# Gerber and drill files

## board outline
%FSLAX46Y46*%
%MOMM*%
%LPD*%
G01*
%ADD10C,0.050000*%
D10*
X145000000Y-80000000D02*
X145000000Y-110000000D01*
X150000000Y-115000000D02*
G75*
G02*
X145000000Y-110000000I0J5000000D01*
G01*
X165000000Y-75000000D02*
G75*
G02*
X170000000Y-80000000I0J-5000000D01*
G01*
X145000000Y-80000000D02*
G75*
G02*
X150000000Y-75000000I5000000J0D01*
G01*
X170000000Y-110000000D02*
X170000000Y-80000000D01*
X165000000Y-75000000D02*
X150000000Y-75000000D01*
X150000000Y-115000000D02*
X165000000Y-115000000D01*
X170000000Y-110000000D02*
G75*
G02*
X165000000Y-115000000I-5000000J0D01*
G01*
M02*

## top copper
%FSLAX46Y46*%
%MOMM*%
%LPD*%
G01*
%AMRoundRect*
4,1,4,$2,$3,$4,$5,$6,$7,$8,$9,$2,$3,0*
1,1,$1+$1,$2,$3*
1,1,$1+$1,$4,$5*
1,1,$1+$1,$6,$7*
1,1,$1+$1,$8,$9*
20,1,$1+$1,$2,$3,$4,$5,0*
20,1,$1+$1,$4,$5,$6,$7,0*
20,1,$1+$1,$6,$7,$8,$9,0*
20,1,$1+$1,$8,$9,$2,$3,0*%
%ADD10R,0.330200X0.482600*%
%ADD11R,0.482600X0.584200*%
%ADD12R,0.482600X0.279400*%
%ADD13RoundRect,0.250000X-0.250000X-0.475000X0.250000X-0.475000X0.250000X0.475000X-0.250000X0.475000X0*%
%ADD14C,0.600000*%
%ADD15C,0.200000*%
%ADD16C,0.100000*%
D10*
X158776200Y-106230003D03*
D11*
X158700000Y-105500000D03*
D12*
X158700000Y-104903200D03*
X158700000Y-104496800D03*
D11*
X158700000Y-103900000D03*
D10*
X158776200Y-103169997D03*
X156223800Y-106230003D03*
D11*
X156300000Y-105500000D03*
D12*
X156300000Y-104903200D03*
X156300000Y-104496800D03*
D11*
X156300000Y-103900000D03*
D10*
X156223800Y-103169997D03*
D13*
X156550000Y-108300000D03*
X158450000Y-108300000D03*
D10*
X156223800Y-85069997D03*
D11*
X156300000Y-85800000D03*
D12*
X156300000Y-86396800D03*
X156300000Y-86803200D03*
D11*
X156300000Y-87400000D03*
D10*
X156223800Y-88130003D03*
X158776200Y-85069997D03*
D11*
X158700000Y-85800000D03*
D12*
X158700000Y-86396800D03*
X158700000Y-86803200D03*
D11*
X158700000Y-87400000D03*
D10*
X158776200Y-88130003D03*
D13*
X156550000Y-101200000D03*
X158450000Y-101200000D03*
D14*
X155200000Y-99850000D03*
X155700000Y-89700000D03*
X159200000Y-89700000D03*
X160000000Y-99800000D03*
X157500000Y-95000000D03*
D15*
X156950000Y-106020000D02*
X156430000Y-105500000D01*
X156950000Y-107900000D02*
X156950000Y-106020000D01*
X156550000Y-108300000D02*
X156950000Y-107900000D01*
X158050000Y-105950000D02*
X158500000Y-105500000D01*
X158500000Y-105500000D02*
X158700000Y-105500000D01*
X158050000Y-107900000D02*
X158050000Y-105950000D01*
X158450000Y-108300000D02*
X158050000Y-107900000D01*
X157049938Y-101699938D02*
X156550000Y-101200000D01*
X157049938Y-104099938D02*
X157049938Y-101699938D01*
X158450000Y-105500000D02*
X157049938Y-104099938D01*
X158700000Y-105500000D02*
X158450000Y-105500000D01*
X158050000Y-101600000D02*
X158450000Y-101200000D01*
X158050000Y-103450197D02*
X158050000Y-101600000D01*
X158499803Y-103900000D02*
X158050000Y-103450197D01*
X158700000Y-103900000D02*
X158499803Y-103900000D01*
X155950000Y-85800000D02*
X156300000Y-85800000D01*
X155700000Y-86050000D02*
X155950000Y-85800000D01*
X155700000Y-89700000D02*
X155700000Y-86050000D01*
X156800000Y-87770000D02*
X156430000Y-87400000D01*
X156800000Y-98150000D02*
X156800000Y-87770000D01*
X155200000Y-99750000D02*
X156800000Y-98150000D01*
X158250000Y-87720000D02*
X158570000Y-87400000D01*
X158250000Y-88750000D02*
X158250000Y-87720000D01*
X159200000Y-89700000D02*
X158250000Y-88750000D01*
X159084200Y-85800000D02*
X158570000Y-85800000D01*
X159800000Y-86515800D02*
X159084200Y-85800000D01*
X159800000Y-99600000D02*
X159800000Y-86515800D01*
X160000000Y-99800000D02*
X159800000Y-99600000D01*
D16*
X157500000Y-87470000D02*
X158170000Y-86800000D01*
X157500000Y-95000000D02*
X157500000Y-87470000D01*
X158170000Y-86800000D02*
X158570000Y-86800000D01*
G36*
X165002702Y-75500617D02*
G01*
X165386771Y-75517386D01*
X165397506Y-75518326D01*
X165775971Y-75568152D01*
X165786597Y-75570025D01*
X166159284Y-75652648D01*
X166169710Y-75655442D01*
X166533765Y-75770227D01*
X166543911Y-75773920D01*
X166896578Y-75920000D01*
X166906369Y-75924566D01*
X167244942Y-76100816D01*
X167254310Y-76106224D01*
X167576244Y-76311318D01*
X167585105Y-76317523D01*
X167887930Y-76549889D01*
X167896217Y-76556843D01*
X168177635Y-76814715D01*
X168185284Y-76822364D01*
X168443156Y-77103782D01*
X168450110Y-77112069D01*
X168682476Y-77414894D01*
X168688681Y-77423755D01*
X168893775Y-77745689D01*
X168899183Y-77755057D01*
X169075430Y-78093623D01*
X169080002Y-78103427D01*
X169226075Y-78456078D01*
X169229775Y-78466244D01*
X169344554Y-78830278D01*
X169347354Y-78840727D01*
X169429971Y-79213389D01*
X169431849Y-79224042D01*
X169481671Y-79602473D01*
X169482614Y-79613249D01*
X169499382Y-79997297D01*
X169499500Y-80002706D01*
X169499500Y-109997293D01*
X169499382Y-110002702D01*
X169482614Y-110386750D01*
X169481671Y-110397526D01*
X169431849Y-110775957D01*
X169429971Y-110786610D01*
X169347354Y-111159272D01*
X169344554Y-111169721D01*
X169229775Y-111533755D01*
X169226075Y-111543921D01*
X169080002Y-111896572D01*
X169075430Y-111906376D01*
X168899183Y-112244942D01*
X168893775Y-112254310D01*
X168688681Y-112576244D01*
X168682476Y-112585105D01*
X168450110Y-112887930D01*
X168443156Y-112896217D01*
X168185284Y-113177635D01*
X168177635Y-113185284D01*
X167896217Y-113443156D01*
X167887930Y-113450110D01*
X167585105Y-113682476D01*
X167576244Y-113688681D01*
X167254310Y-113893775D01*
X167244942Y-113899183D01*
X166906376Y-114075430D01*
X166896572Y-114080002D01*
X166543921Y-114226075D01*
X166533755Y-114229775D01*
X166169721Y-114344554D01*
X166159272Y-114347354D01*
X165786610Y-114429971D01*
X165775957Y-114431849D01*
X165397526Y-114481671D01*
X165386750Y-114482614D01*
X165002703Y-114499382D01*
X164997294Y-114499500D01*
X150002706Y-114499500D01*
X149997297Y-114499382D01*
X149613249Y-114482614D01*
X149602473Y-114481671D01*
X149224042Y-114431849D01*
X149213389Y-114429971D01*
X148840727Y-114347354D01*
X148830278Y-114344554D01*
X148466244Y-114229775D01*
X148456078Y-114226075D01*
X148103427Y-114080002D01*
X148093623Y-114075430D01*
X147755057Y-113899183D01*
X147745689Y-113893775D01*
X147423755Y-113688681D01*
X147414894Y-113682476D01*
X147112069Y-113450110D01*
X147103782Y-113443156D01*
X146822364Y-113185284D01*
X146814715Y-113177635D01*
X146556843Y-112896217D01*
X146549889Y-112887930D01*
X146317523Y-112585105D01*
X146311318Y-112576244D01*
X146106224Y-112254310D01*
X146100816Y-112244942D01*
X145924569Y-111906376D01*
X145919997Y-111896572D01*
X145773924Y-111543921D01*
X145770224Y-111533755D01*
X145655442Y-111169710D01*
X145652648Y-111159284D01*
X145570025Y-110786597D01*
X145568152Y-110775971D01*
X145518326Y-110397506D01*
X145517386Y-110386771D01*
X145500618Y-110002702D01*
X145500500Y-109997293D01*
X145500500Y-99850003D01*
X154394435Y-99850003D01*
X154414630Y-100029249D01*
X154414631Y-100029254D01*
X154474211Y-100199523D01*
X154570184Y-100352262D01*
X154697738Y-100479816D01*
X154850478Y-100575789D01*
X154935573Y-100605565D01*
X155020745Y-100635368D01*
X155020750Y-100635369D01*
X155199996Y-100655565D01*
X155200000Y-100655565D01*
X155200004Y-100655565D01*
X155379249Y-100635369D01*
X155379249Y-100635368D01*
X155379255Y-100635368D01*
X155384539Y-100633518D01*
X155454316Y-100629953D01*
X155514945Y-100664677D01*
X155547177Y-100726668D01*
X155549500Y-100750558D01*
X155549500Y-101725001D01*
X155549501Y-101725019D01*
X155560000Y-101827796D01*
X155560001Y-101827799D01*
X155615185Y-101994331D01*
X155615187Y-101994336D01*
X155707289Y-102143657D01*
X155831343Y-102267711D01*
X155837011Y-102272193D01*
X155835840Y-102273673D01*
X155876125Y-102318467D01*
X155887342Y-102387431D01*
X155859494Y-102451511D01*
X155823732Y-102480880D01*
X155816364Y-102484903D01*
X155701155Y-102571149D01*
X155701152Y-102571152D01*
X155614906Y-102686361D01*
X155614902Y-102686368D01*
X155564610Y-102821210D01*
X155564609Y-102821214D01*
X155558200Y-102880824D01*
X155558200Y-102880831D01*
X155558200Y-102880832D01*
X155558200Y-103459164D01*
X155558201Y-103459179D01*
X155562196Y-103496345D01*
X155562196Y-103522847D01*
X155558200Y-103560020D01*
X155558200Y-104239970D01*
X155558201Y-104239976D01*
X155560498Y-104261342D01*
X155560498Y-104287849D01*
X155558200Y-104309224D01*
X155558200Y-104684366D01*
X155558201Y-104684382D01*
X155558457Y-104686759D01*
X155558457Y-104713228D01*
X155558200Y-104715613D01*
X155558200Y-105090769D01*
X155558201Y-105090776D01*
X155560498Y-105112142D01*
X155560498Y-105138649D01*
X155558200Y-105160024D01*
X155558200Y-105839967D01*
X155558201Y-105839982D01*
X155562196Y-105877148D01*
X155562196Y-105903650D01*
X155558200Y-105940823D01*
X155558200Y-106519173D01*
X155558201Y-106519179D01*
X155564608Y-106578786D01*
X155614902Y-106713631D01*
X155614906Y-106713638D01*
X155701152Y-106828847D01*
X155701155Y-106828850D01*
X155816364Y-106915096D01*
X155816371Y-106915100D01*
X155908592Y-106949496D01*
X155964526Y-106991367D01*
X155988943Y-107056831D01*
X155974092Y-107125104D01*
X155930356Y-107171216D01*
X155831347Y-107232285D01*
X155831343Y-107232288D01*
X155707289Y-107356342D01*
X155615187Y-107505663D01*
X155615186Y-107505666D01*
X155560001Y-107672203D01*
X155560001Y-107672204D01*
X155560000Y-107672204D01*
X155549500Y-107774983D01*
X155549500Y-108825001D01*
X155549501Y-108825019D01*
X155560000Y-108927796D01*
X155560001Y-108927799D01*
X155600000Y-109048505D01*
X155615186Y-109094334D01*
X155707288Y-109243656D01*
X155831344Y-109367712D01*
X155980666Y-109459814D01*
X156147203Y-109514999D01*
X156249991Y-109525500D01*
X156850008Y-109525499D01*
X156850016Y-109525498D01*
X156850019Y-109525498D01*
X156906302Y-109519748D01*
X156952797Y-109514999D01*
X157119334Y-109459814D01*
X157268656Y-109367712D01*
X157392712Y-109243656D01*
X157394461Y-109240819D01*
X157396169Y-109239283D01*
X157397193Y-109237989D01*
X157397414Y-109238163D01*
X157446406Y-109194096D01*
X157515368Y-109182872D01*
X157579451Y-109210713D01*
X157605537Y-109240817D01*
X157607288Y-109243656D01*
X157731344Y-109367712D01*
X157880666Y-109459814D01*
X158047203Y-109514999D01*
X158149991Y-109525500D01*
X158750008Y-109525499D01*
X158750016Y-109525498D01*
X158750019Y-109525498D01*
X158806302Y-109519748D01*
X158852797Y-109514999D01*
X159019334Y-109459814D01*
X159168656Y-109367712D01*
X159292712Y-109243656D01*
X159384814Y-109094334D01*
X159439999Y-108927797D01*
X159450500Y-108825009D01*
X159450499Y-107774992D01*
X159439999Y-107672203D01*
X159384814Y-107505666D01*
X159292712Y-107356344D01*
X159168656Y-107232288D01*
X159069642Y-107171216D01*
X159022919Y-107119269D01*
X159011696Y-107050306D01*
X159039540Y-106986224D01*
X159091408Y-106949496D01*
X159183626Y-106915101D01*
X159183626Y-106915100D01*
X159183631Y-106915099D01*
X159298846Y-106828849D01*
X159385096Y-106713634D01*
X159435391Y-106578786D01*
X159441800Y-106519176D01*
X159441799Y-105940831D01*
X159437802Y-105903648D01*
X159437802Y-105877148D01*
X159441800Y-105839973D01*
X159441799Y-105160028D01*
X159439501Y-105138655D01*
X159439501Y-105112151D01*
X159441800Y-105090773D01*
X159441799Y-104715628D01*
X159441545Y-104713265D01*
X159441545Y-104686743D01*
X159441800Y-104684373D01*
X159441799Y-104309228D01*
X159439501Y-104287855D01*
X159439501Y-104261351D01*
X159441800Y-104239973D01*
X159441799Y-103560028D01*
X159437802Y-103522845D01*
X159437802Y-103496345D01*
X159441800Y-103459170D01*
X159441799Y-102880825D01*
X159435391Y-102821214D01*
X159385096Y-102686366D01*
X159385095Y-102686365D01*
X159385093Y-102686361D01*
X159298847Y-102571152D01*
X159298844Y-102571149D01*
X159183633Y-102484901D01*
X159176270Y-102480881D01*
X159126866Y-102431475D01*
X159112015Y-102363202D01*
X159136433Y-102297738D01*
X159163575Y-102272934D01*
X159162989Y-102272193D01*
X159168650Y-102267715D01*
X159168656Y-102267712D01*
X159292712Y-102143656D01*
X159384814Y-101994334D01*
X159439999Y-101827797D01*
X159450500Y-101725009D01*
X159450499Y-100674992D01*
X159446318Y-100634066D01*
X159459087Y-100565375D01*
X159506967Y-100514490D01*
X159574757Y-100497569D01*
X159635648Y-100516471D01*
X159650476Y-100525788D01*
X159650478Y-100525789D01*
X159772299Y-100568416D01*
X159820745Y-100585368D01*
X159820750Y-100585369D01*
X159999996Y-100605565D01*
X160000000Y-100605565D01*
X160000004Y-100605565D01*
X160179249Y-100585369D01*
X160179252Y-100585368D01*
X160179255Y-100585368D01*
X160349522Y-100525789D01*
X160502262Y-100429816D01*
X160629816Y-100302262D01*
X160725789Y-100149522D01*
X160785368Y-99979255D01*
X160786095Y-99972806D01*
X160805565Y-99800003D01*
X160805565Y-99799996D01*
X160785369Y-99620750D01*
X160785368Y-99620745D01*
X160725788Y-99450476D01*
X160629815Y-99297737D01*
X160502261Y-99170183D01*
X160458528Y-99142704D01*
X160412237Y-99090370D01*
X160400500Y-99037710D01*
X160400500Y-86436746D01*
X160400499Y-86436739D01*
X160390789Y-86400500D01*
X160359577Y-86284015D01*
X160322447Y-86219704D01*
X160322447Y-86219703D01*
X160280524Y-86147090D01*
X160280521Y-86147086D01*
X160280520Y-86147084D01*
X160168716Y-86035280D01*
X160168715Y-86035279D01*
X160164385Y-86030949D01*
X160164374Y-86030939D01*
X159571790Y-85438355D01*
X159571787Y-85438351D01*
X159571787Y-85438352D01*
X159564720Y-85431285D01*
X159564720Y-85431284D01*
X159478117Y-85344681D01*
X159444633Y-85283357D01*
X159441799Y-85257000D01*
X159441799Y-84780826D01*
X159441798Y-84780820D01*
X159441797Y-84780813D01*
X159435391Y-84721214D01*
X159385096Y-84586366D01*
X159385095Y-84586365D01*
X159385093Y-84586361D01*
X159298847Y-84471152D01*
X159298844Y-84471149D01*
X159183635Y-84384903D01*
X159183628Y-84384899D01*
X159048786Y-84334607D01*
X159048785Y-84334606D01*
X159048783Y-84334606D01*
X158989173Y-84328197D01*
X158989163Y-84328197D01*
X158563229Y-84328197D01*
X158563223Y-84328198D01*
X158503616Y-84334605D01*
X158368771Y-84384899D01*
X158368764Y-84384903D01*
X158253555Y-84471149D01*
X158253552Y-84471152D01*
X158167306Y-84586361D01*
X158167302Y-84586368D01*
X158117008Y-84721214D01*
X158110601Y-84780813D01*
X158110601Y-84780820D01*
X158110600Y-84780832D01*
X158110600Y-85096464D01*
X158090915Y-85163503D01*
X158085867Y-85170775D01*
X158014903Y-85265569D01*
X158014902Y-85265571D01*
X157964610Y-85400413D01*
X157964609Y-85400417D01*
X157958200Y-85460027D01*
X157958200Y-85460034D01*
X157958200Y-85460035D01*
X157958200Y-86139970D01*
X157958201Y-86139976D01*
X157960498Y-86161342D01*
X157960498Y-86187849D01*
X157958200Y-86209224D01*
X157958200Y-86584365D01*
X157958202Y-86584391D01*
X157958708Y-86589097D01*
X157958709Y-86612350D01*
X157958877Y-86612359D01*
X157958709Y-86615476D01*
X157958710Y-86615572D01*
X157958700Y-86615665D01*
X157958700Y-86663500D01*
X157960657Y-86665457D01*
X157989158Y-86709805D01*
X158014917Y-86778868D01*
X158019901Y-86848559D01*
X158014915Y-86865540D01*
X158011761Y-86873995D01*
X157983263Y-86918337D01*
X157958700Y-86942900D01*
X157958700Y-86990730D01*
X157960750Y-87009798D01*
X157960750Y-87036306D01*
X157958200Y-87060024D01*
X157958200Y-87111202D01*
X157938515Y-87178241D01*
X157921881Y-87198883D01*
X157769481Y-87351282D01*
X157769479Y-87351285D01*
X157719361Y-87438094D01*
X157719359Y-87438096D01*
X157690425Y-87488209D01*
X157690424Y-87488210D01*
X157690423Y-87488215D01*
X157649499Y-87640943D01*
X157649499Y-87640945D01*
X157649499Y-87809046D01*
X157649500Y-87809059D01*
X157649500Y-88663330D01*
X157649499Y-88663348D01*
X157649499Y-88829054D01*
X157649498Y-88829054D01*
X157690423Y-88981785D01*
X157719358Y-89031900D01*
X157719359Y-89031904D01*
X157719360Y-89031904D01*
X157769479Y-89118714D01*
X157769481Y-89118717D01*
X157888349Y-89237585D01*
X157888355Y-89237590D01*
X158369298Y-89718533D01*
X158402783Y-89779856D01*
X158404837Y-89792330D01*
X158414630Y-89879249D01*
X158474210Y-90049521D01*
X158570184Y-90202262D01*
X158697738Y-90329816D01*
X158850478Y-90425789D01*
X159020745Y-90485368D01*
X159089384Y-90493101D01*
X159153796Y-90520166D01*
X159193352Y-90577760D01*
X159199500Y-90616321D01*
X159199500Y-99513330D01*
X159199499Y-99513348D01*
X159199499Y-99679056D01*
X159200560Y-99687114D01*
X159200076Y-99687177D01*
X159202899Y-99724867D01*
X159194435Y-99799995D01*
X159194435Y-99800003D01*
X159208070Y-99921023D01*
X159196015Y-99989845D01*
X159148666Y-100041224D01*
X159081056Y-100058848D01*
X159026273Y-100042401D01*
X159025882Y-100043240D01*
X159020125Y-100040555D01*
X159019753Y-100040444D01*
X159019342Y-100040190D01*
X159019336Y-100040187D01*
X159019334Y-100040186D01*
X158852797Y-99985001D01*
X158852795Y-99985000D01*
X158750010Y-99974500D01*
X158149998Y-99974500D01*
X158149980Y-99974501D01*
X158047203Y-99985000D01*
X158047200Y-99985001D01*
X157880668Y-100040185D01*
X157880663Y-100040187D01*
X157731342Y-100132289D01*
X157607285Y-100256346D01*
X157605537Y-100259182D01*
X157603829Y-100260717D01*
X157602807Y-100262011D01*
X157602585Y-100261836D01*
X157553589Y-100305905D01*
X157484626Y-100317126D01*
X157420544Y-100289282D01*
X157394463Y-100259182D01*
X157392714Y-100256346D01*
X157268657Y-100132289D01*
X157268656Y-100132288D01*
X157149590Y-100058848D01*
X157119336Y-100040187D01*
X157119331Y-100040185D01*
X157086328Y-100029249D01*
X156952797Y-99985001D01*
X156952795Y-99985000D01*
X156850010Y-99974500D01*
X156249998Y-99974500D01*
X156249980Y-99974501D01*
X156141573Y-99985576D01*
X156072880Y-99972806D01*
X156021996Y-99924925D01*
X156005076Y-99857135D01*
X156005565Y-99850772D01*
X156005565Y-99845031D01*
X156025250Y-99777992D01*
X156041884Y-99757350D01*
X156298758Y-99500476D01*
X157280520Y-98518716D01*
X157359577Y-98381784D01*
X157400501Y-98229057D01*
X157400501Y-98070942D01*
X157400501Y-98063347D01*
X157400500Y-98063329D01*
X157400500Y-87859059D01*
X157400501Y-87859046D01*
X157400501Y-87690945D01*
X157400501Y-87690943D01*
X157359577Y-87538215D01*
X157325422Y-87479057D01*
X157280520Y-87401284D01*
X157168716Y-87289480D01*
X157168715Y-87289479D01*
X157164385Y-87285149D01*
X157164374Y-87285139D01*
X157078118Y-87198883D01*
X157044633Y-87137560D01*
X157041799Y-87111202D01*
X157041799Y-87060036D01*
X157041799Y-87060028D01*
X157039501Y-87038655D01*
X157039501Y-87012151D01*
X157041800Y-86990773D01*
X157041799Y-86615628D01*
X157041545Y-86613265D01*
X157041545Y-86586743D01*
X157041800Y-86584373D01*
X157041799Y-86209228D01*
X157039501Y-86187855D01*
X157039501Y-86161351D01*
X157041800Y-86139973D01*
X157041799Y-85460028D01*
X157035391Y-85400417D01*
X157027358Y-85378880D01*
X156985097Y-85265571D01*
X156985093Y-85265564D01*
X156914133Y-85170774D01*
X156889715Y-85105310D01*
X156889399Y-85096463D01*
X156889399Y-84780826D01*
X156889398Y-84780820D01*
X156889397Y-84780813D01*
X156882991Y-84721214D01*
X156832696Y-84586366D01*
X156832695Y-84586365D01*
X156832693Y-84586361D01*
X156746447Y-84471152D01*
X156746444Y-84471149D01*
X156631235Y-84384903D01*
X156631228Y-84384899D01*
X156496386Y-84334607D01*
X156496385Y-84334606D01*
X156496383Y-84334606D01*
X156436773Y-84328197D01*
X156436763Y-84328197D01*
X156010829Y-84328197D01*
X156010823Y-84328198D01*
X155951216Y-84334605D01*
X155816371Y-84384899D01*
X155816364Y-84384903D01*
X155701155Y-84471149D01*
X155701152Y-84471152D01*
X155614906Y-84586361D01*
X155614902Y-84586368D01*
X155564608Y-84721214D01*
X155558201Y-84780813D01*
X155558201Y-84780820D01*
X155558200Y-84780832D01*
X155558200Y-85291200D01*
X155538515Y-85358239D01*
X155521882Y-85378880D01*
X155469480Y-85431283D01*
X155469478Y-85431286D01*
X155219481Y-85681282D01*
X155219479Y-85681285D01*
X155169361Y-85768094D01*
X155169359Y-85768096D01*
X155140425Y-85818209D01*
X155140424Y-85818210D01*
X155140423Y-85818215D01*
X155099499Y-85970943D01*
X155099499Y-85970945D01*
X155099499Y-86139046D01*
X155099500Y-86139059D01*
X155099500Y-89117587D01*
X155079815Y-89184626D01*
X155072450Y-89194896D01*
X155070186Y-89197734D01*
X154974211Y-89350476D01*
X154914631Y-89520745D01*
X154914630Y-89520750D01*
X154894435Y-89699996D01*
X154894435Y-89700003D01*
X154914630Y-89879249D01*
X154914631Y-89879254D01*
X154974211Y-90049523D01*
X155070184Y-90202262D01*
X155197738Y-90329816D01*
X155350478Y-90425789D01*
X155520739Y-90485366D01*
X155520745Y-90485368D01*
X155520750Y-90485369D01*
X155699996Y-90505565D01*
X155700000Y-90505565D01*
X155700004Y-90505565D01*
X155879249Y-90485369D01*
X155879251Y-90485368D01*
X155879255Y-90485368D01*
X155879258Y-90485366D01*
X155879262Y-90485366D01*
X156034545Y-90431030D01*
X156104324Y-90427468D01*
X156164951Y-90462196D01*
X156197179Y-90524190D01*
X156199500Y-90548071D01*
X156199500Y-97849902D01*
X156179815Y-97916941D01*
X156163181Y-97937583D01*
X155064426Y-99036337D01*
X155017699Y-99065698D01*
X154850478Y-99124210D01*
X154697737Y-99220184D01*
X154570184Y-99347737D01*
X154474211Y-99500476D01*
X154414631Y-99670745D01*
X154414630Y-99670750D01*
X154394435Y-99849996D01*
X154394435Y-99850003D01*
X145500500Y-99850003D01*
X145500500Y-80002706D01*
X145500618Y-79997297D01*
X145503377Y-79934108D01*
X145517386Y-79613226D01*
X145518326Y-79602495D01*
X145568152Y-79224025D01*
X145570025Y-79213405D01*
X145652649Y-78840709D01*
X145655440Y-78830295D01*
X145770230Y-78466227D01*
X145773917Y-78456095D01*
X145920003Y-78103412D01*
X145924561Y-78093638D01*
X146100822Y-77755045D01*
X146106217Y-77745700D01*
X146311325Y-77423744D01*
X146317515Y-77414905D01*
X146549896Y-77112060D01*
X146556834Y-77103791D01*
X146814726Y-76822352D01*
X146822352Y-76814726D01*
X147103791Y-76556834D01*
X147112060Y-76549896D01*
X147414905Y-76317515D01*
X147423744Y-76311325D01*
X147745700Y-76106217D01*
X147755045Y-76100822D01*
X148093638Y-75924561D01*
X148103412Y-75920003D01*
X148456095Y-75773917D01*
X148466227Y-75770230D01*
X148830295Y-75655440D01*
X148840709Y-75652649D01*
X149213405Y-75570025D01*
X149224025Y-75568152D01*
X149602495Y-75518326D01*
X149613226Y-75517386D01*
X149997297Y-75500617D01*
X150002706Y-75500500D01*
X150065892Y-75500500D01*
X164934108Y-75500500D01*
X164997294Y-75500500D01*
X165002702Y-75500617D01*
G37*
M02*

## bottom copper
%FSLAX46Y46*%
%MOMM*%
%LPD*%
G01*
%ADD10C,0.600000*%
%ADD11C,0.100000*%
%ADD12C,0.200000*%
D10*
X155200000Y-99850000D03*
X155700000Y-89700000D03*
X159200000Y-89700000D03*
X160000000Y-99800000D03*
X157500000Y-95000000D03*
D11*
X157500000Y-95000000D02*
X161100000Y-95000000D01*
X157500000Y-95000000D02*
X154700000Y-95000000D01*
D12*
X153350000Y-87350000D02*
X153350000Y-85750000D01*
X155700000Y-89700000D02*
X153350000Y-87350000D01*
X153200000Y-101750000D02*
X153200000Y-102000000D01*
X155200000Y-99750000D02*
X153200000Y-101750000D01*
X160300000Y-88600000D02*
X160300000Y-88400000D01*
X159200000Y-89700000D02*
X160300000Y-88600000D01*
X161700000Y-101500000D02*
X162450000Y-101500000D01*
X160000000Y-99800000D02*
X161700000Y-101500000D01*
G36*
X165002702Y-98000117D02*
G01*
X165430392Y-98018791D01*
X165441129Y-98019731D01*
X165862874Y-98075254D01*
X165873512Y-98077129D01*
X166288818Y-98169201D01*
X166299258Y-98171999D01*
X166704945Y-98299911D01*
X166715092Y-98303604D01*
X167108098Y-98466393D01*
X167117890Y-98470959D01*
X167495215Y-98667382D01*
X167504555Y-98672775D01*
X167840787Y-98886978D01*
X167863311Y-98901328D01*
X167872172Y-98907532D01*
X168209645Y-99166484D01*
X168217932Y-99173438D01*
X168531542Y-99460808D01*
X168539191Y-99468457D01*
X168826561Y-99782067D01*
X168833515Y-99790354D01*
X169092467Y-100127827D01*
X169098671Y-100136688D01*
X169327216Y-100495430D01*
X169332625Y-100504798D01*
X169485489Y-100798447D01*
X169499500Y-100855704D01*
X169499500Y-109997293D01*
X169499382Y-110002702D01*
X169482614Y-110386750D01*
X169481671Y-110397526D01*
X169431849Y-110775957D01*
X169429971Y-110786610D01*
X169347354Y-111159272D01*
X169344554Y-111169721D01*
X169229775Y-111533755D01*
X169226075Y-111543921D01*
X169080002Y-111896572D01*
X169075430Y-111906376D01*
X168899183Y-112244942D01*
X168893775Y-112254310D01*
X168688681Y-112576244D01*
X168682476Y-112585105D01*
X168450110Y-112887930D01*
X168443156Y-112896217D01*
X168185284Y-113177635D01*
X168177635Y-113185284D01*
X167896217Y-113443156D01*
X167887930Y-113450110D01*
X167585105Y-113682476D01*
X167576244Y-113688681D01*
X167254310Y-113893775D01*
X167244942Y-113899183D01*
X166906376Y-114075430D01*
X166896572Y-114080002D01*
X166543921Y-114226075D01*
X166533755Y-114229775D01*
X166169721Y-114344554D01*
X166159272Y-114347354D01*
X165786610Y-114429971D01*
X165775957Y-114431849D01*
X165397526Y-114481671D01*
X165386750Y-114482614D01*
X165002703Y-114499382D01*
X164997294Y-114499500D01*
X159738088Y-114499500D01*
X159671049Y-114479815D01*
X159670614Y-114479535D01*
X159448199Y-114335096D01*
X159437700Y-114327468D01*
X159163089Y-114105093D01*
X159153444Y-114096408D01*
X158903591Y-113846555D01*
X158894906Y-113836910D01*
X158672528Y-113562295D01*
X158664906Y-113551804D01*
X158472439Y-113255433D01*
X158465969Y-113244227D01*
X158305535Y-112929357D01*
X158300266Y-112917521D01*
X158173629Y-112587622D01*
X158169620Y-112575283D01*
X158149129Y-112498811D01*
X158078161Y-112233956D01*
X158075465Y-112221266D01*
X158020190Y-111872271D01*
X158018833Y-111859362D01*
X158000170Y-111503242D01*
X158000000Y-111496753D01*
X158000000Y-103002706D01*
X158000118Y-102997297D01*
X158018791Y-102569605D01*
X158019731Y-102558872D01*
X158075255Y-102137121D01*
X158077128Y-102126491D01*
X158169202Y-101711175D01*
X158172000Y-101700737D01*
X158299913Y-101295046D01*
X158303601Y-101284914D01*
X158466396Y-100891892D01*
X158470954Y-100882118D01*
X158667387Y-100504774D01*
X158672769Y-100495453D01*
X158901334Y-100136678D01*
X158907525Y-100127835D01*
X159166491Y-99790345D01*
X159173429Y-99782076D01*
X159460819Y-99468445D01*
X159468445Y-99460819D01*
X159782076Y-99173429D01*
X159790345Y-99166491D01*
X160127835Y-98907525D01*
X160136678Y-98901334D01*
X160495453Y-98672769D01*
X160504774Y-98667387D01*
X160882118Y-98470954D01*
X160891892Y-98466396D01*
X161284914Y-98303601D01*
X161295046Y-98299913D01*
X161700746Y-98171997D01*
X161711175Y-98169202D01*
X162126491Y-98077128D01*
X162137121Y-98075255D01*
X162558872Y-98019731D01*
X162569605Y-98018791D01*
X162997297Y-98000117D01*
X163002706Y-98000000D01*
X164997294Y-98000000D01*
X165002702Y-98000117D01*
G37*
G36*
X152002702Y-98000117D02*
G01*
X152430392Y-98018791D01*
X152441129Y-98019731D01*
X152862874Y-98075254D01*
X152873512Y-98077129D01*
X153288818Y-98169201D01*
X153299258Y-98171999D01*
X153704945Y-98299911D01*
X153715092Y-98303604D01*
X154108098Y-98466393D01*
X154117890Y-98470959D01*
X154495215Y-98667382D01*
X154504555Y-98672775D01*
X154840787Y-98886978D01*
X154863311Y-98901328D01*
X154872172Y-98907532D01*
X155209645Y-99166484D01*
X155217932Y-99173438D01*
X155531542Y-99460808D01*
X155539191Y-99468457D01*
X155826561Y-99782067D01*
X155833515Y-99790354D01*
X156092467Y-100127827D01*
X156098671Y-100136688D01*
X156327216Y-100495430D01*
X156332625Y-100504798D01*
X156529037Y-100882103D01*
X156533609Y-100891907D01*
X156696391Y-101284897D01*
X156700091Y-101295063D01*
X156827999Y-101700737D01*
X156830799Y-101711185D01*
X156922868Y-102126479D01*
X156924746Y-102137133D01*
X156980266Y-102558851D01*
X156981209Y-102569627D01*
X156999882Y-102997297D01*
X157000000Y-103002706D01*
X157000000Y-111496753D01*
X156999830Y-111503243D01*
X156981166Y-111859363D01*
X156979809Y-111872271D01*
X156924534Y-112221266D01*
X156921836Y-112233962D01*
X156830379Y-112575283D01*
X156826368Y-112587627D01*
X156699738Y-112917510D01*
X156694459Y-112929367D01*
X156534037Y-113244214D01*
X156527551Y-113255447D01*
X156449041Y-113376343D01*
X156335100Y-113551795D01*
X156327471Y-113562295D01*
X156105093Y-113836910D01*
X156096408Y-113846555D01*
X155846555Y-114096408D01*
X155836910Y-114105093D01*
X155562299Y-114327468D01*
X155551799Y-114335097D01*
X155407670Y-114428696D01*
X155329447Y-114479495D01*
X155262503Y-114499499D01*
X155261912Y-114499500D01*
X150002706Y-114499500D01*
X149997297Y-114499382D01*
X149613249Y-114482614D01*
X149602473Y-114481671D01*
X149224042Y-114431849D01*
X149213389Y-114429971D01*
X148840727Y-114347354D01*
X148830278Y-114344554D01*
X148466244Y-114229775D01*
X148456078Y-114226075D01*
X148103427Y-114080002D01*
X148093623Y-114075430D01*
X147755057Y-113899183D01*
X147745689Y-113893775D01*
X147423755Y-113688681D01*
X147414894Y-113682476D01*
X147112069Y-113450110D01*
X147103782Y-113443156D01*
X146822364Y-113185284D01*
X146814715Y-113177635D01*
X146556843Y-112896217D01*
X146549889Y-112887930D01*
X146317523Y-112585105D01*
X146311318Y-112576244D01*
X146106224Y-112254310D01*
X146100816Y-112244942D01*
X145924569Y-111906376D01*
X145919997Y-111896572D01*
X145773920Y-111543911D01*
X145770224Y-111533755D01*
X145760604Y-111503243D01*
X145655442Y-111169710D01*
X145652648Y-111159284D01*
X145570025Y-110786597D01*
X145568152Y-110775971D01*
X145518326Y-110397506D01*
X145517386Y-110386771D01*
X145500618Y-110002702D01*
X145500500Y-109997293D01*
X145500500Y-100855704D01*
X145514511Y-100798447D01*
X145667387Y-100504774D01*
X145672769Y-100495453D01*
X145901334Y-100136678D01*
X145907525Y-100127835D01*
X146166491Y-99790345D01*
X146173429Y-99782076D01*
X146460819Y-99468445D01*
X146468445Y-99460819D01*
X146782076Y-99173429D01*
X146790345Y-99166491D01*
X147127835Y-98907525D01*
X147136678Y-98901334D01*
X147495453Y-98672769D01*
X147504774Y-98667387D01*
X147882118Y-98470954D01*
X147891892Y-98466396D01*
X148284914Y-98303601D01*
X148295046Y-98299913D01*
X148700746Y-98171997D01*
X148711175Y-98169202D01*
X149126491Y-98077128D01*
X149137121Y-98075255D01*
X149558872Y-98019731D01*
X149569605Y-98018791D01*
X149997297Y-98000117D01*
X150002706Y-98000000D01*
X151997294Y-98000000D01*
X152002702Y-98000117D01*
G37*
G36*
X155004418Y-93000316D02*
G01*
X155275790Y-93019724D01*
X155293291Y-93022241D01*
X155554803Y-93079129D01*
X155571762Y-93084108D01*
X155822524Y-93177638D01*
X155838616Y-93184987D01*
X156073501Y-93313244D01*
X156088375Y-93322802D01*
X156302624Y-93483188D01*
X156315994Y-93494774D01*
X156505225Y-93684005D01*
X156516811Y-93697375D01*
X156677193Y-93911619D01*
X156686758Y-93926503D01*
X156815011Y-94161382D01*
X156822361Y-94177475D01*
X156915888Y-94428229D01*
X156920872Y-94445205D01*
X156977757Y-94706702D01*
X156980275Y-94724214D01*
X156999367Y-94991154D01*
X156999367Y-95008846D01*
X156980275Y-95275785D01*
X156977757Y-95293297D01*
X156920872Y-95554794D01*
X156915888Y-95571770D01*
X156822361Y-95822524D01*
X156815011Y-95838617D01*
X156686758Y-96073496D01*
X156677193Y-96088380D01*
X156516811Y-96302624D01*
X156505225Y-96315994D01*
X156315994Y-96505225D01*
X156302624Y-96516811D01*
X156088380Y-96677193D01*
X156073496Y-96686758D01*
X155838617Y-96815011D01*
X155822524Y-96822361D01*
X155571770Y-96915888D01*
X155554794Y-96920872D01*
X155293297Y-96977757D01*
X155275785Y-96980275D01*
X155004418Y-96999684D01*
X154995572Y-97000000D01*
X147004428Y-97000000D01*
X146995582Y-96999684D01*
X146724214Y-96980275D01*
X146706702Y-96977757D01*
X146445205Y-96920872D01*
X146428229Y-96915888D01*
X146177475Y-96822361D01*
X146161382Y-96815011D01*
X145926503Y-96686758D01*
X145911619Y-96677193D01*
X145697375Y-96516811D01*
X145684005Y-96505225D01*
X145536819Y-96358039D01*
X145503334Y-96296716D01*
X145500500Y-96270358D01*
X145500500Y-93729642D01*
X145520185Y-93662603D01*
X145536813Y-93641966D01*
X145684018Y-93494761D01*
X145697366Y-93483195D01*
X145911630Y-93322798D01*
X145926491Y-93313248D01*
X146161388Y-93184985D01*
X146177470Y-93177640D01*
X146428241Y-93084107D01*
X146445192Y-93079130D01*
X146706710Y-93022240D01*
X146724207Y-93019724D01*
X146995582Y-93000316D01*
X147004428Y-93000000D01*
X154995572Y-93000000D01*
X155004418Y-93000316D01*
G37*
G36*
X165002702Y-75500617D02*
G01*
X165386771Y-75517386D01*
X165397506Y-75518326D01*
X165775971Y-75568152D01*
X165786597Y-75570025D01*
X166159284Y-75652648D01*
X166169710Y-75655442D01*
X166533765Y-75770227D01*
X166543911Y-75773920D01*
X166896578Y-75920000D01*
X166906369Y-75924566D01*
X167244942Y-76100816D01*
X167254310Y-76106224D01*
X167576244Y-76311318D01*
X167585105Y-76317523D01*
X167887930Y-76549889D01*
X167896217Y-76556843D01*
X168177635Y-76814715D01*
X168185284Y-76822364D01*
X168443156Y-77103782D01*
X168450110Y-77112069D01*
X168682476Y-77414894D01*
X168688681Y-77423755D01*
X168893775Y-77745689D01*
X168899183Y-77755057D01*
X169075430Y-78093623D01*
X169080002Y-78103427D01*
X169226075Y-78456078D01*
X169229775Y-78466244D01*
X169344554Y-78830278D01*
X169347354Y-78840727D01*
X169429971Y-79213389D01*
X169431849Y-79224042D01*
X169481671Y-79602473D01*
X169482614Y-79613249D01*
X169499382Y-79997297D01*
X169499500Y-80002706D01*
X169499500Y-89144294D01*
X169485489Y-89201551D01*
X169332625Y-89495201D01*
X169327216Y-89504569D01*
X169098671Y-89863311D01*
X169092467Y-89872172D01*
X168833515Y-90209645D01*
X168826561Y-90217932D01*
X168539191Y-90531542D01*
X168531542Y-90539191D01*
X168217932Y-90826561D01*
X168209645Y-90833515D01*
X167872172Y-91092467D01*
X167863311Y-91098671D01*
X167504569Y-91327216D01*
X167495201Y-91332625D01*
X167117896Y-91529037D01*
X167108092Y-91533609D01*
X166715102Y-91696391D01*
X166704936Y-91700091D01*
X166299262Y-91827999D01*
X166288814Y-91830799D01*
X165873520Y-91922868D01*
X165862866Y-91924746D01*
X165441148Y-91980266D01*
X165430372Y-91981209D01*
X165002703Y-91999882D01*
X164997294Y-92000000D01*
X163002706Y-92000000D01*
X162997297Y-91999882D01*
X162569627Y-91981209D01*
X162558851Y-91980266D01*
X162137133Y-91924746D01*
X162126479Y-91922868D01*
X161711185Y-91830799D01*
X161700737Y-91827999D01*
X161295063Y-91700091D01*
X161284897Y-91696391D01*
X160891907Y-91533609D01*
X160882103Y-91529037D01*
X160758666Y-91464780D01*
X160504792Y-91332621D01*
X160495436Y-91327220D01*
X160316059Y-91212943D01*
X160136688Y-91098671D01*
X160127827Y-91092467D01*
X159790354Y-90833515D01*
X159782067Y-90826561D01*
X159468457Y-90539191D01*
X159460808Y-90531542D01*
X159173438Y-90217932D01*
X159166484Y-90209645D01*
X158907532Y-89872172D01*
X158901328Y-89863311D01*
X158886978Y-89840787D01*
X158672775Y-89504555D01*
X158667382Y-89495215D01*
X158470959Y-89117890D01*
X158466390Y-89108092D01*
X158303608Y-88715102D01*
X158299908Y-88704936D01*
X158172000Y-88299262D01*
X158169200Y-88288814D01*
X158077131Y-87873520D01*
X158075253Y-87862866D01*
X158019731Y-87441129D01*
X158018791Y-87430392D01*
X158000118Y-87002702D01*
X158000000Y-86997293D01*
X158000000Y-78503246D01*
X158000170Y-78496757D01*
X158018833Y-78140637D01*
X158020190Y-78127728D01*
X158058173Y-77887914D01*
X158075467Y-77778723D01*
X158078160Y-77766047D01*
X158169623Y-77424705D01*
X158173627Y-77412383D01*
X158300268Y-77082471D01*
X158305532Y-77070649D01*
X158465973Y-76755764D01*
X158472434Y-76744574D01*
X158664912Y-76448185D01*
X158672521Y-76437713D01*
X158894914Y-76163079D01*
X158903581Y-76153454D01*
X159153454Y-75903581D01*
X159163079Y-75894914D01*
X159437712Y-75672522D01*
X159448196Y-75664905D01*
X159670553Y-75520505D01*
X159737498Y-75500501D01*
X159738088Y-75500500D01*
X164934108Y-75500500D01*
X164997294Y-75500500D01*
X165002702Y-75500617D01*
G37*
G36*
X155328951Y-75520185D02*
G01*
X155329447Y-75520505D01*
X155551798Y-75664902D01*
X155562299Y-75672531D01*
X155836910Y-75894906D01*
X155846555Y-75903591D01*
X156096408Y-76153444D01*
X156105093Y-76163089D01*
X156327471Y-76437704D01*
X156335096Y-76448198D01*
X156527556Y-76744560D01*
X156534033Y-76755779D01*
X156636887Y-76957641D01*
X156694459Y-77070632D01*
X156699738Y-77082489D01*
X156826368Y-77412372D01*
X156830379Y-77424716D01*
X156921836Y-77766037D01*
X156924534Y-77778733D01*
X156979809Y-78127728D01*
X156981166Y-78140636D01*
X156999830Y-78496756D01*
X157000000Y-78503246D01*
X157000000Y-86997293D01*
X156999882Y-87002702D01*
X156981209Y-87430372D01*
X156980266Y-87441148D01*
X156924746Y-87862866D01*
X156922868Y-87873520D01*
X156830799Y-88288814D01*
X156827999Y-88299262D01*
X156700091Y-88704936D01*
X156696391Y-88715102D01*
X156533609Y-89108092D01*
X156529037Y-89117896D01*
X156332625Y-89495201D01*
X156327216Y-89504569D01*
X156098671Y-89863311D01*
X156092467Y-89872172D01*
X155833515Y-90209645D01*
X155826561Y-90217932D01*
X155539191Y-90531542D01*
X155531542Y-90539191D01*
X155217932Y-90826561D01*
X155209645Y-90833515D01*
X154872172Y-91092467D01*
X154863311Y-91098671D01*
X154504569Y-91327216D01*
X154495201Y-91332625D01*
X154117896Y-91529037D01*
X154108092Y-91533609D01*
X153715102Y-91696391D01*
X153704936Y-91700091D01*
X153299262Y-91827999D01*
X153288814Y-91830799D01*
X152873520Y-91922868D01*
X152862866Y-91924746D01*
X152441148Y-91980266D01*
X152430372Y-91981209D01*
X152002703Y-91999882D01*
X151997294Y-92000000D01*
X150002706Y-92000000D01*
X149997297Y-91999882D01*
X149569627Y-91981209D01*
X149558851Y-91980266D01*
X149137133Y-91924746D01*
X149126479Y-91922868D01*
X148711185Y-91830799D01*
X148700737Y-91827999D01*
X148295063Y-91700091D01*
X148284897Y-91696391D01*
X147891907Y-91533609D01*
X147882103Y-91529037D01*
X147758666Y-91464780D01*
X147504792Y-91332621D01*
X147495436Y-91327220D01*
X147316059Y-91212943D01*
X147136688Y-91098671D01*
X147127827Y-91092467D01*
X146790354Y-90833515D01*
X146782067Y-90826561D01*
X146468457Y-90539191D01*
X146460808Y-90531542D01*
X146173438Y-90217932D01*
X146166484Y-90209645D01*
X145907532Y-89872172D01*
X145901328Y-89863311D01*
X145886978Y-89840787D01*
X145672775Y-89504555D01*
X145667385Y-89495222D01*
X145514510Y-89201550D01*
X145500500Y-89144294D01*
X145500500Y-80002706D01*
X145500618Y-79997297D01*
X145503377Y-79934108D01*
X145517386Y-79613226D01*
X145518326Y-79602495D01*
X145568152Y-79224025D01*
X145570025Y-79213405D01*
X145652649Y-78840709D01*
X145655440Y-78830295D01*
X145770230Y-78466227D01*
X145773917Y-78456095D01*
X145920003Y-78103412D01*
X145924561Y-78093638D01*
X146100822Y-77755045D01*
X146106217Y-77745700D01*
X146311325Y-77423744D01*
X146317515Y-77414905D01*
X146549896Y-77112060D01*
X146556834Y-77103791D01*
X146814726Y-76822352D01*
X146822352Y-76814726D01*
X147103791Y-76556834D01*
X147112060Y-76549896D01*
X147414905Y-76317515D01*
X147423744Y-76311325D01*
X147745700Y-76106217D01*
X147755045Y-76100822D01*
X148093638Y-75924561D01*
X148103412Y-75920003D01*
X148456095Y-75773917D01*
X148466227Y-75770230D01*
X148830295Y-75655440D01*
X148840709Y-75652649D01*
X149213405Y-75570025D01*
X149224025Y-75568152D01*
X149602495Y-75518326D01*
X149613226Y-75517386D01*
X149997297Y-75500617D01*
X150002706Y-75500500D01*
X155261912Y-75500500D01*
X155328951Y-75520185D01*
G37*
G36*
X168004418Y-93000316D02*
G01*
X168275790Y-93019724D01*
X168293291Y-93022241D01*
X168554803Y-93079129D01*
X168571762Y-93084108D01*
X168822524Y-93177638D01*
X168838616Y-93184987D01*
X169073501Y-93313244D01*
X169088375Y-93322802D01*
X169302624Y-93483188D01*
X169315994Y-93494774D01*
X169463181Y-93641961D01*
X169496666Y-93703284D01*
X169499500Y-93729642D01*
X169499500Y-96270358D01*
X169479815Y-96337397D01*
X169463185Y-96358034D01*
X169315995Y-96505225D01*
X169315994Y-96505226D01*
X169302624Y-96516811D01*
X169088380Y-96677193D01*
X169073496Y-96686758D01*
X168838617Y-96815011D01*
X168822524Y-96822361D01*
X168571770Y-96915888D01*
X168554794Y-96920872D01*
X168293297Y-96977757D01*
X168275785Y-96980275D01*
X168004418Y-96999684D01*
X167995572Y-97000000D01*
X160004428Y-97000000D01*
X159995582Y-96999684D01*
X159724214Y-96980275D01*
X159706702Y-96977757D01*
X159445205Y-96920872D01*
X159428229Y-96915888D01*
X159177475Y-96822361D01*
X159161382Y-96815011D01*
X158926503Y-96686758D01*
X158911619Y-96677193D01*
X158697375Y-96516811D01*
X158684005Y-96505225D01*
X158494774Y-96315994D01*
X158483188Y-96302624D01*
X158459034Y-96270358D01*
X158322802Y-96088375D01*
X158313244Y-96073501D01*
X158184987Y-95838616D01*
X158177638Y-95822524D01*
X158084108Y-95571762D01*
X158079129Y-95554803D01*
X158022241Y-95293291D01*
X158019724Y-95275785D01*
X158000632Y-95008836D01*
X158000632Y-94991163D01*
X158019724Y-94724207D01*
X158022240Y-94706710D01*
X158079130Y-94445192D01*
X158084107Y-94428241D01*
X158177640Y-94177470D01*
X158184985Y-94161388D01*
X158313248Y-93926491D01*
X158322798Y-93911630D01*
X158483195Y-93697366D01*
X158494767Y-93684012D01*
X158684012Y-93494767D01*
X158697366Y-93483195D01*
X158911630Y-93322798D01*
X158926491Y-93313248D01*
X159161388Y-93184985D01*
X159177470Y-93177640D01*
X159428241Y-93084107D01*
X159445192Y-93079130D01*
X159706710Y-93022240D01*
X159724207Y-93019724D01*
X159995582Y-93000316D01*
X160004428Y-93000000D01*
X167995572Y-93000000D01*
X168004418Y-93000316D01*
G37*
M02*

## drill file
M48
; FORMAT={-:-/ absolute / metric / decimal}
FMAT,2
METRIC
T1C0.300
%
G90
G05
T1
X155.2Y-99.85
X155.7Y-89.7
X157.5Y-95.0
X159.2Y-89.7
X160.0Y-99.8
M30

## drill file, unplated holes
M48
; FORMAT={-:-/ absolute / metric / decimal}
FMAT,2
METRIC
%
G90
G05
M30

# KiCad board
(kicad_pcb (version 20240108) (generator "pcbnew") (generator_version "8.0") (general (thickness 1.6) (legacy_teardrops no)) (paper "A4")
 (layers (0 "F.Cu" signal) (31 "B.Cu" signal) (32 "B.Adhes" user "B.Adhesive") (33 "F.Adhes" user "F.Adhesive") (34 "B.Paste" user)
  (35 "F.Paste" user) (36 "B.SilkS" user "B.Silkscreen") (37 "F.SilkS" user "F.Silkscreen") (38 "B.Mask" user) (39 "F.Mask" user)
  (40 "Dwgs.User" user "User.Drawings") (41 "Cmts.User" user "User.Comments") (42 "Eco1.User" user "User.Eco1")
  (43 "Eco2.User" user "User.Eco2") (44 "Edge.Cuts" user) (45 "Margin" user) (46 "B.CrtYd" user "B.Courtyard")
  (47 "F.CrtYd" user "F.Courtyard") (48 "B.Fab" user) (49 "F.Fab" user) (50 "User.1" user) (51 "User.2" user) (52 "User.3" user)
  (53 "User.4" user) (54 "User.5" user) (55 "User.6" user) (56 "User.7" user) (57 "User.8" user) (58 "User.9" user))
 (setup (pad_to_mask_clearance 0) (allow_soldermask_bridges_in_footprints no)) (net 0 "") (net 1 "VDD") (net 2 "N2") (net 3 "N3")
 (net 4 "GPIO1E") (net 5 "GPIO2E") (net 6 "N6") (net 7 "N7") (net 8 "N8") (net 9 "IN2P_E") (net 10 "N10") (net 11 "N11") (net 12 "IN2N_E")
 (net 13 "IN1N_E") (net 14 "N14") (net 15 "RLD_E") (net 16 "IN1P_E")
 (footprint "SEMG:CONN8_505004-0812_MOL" (layer "F.Cu") (at 157.5 104.7 -90)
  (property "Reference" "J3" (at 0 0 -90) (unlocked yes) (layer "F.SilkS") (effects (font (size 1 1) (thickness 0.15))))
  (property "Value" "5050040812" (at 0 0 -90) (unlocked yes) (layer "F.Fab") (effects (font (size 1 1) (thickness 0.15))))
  (pad "1" smd rect (at 0.8 -1.2 270) (size 0.5842 0.4826) (layers "F.Cu" "F.Paste" "F.Mask") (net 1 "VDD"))
  (pad "2" smd rect (at 0.2032 -1.2 270) (size 0.2794 0.4826) (layers "F.Cu" "F.Paste" "F.Mask") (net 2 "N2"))
  (pad "3" smd rect (at -0.2032 -1.2 270) (size 0.2794 0.4826) (layers "F.Cu" "F.Paste" "F.Mask") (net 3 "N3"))
  (pad "4" smd rect (at -0.8 -1.2 270) (size 0.5842 0.4826) (layers "F.Cu" "F.Paste" "F.Mask") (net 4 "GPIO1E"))
  (pad "5" smd rect (at 0.8 1.2 270) (size 0.5842 0.4826) (layers "F.Cu" "F.Paste" "F.Mask") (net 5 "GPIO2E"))
  (pad "6" smd rect (at 0.2032 1.2 270) (size 0.2794 0.4826) (layers "F.Cu" "F.Paste" "F.Mask") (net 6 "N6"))
  (pad "7" smd rect (at -0.2032 1.2 270) (size 0.2794 0.4826) (layers "F.Cu" "F.Paste" "F.Mask") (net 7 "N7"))
  (pad "8" smd rect (at -0.8 1.2 270) (size 0.5842 0.4826) (layers "F.Cu" "F.Paste" "F.Mask") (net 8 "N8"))
  (pad "9" smd rect (at 1.530003 -1.2762 270) (size 0.4826 0.3302) (layers "F.Cu" "F.Paste" "F.Mask"))
  (pad "10" smd rect (at -1.530003 -1.2762 270) (size 0.4826 0.3302) (layers "F.Cu" "F.Paste" "F.Mask"))
  (pad "11" smd rect (at 1.530003 1.2762 270) (size 0.4826 0.3302) (layers "F.Cu" "F.Paste" "F.Mask"))
  (pad "12" smd rect (at -1.530003 1.2762 270) (size 0.4826 0.3302) (layers "F.Cu" "F.Paste" "F.Mask")))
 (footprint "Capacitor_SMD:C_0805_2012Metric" (layer "F.Cu") (at 157.5 108.3)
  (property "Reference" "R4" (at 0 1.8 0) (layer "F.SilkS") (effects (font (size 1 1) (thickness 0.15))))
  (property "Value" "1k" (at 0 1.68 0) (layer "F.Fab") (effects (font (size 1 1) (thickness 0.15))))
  (pad "1" smd roundrect (at -0.95 0) (size 1 1.45) (layers "F.Cu" "F.Paste" "F.Mask") (roundrect_rratio 0.25) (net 5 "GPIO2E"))
  (pad "2" smd roundrect (at 0.95 0) (size 1 1.45) (layers "F.Cu" "F.Paste" "F.Mask") (roundrect_rratio 0.25) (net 1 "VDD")))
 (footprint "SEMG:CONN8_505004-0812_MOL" (layer "F.Cu") (at 157.5 86.6 90)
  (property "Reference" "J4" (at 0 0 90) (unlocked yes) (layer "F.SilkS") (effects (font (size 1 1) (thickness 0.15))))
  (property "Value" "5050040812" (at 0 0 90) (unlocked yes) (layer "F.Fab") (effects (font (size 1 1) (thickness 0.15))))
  (pad "1" smd rect (at 0.8 -1.2 90) (size 0.5842 0.4826) (layers "F.Cu" "F.Paste" "F.Mask") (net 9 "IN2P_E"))
  (pad "2" smd rect (at 0.2032 -1.2 90) (size 0.2794 0.4826) (layers "F.Cu" "F.Paste" "F.Mask") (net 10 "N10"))
  (pad "3" smd rect (at -0.2032 -1.2 90) (size 0.2794 0.4826) (layers "F.Cu" "F.Paste" "F.Mask") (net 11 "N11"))
  (pad "4" smd rect (at -0.8 -1.2 90) (size 0.5842 0.4826) (layers "F.Cu" "F.Paste" "F.Mask") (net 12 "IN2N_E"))
  (pad "5" smd rect (at 0.8 1.2 90) (size 0.5842 0.4826) (layers "F.Cu" "F.Paste" "F.Mask") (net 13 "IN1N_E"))
  (pad "6" smd rect (at 0.2032 1.2 90) (size 0.2794 0.4826) (layers "F.Cu" "F.Paste" "F.Mask") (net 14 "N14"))
  (pad "7" smd rect (at -0.2032 1.2 90) (size 0.2794 0.4826) (layers "F.Cu" "F.Paste" "F.Mask") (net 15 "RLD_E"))
  (pad "8" smd rect (at -0.8 1.2 90) (size 0.5842 0.4826) (layers "F.Cu" "F.Paste" "F.Mask") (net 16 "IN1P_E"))
  (pad "9" smd rect (at 1.530003 -1.2762 90) (size 0.4826 0.3302) (layers "F.Cu" "F.Paste" "F.Mask"))
  (pad "10" smd rect (at -1.530003 -1.2762 90) (size 0.4826 0.3302) (layers "F.Cu" "F.Paste" "F.Mask"))
  (pad "11" smd rect (at 1.530003 1.2762 90) (size 0.4826 0.3302) (layers "F.Cu" "F.Paste" "F.Mask"))
  (pad "12" smd rect (at -1.530003 1.2762 90) (size 0.4826 0.3302) (layers "F.Cu" "F.Paste" "F.Mask")))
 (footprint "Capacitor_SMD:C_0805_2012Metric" (layer "F.Cu") (at 157.5 101.2)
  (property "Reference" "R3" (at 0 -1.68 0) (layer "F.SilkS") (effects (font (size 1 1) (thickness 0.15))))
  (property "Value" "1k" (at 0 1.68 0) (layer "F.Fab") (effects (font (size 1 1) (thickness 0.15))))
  (pad "1" smd roundrect (at -0.95 0) (size 1 1.45) (layers "F.Cu" "F.Paste" "F.Mask") (roundrect_rratio 0.25) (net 1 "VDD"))
  (pad "2" smd roundrect (at 0.95 0) (size 1 1.45) (layers "F.Cu" "F.Paste" "F.Mask") (roundrect_rratio 0.25) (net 4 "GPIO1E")))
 (gr_line (start 145 80) (end 145 110) (stroke (width 0.05) (type default)) (layer "Edge.Cuts"))
 (gr_arc (start 150 115) (mid 146.464466 113.535534) (end 145 110) (stroke (width 0.05) (type default)) (layer "Edge.Cuts"))
 (gr_arc (start 165 75) (mid 168.535534 76.464466) (end 170 80) (stroke (width 0.05) (type default)) (layer "Edge.Cuts"))
 (gr_arc (start 145 80) (mid 146.464466 76.464466) (end 150 75) (stroke (width 0.05) (type default)) (layer "Edge.Cuts"))
 (gr_line (start 170 110) (end 170 80) (stroke (width 0.05) (type default)) (layer "Edge.Cuts"))
 (gr_line (start 165 75) (end 150 75) (stroke (width 0.05) (type default)) (layer "Edge.Cuts"))
 (gr_line (start 150 115) (end 165 115) (stroke (width 0.05) (type default)) (layer "Edge.Cuts"))
 (gr_arc (start 170 110) (mid 168.535534 113.535534) (end 165 115) (stroke (width 0.05) (type default)) (layer "Edge.Cuts"))
 (segment (start 156.8 98.15) (end 156.8 87.77) (width 0.2) (layer "F.Cu") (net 12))
 (segment (start 155.2 99.75) (end 156.8 98.15) (width 0.2) (layer "F.Cu") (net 12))
 (segment (start 156.8 87.77) (end 156.43 87.4) (width 0.2) (layer "F.Cu") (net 12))
 (via (at 155.2 99.85) (size 0.6) (drill 0.3) (layers "F.Cu" "B.Cu") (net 12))
 (segment (start 155.2 99.75) (end 153.2 101.75) (width 0.2) (layer "B.Cu") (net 12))
 (segment (start 153.2 101.75) (end 153.2 102) (width 0.2) (layer "B.Cu") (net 12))
 (segment (start 155.95 85.8) (end 156.3 85.8) (width 0.2) (layer "F.Cu") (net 9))
 (segment (start 155.7 86.05) (end 155.95 85.8) (width 0.2) (layer "F.Cu") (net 9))
 (segment (start 155.7 89.7) (end 155.7 86.05) (width 0.2) (layer "F.Cu") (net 9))
 (via (at 155.7 89.7) (size 0.6) (drill 0.3) (layers "F.Cu" "B.Cu") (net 9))
 (segment (start 153.35 87.35) (end 153.35 85.75) (width 0.2) (layer "B.Cu") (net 9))
 (segment (start 155.7 89.7) (end 153.35 87.35) (width 0.2) (layer "B.Cu") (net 9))
 (segment (start 158.25 87.72) (end 158.57 87.4) (width 0.2) (layer "F.Cu") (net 16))
 (segment (start 159.2 89.7) (end 158.25 88.75) (width 0.2) (layer "F.Cu") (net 16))
 (segment (start 158.25 88.75) (end 158.25 87.72) (width 0.2) (layer "F.Cu") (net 16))
 (via (at 159.2 89.7) (size 0.6) (drill 0.3) (layers "F.Cu" "B.Cu") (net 16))
 (segment (start 160.3 88.6) (end 160.3 88.4) (width 0.2) (layer "B.Cu") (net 16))
 (segment (start 159.2 89.7) (end 160.3 88.6) (width 0.2) (layer "B.Cu") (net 16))
 (segment (start 159.8 99.6) (end 159.8 86.5158) (width 0.2) (layer "F.Cu") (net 13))
 (segment (start 159.8 86.5158) (end 159.0842 85.8) (width 0.2) (layer "F.Cu") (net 13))
 (segment (start 159.0842 85.8) (end 158.57 85.8) (width 0.2) (layer "F.Cu") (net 13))
 (segment (start 160 99.8) (end 159.8 99.6) (width 0.2) (layer "F.Cu") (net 13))
 (via (at 160 99.8) (size 0.6) (drill 0.3) (layers "F.Cu" "B.Cu") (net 13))
 (segment (start 160 99.8) (end 161.7 101.5) (width 0.2) (layer "B.Cu") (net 13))
 (segment (start 161.7 101.5) (end 162.45 101.5) (width 0.2) (layer "B.Cu") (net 13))
 (segment (start 157.5 87.47) (end 158.17 86.8) (width 0.1) (layer "F.Cu") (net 15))
 (segment (start 157.5 95) (end 157.5 87.47) (width 0.1) (layer "F.Cu") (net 15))
 (segment (start 158.17 86.8) (end 158.57 86.8) (width 0.1) (layer "F.Cu") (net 15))
 (via (at 157.5 95) (size 0.6) (drill 0.3) (layers "F.Cu" "B.Cu") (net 15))
 (segment (start 157.5 95) (end 161.1 95) (width 0.1) (layer "B.Cu") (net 15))
 (segment (start 157.5 95) (end 154.7 95) (width 0.1) (layer "B.Cu") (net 15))
 (segment (start 156.95 106.02) (end 156.43 105.5) (width 0.2) (layer "F.Cu") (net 5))
 (segment (start 156.55 108.3) (end 156.95 107.9) (width 0.2) (layer "F.Cu") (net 5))
 (segment (start 156.95 107.9) (end 156.95 106.02) (width 0.2) (layer "F.Cu") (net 5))
 (segment (start 158.7 105.5) (end 158.45 105.5) (width 0.2) (layer "F.Cu") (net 1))
 (segment (start 158.45 108.3) (end 158.05 107.9) (width 0.2) (layer "F.Cu") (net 1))
 (segment (start 157.049938 104.099938) (end 157.049938 101.699938) (width 0.2) (layer "F.Cu") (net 1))
 (segment (start 158.5 105.5) (end 158.7 105.5) (width 0.2) (layer "F.Cu") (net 1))
 (segment (start 158.05 107.9) (end 158.05 105.95) (width 0.2) (layer "F.Cu") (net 1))
 (segment (start 157.049938 101.699938) (end 156.55 101.2) (width 0.2) (layer "F.Cu") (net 1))
 (segment (start 158.45 105.5) (end 157.049938 104.099938) (width 0.2) (layer "F.Cu") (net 1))
 (segment (start 158.05 105.95) (end 158.5 105.5) (width 0.2) (layer "F.Cu") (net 1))
 (segment (start 158.499803 103.9) (end 158.05 103.450197) (width 0.2) (layer "F.Cu") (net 4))
 (segment (start 158.05 103.450197) (end 158.05 101.6) (width 0.2) (layer "F.Cu") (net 4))
 (segment (start 158.05 101.6) (end 158.45 101.2) (width 0.2) (layer "F.Cu") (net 4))
 (segment (start 158.7 103.9) (end 158.499803 103.9) (width 0.2) (layer "F.Cu") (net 4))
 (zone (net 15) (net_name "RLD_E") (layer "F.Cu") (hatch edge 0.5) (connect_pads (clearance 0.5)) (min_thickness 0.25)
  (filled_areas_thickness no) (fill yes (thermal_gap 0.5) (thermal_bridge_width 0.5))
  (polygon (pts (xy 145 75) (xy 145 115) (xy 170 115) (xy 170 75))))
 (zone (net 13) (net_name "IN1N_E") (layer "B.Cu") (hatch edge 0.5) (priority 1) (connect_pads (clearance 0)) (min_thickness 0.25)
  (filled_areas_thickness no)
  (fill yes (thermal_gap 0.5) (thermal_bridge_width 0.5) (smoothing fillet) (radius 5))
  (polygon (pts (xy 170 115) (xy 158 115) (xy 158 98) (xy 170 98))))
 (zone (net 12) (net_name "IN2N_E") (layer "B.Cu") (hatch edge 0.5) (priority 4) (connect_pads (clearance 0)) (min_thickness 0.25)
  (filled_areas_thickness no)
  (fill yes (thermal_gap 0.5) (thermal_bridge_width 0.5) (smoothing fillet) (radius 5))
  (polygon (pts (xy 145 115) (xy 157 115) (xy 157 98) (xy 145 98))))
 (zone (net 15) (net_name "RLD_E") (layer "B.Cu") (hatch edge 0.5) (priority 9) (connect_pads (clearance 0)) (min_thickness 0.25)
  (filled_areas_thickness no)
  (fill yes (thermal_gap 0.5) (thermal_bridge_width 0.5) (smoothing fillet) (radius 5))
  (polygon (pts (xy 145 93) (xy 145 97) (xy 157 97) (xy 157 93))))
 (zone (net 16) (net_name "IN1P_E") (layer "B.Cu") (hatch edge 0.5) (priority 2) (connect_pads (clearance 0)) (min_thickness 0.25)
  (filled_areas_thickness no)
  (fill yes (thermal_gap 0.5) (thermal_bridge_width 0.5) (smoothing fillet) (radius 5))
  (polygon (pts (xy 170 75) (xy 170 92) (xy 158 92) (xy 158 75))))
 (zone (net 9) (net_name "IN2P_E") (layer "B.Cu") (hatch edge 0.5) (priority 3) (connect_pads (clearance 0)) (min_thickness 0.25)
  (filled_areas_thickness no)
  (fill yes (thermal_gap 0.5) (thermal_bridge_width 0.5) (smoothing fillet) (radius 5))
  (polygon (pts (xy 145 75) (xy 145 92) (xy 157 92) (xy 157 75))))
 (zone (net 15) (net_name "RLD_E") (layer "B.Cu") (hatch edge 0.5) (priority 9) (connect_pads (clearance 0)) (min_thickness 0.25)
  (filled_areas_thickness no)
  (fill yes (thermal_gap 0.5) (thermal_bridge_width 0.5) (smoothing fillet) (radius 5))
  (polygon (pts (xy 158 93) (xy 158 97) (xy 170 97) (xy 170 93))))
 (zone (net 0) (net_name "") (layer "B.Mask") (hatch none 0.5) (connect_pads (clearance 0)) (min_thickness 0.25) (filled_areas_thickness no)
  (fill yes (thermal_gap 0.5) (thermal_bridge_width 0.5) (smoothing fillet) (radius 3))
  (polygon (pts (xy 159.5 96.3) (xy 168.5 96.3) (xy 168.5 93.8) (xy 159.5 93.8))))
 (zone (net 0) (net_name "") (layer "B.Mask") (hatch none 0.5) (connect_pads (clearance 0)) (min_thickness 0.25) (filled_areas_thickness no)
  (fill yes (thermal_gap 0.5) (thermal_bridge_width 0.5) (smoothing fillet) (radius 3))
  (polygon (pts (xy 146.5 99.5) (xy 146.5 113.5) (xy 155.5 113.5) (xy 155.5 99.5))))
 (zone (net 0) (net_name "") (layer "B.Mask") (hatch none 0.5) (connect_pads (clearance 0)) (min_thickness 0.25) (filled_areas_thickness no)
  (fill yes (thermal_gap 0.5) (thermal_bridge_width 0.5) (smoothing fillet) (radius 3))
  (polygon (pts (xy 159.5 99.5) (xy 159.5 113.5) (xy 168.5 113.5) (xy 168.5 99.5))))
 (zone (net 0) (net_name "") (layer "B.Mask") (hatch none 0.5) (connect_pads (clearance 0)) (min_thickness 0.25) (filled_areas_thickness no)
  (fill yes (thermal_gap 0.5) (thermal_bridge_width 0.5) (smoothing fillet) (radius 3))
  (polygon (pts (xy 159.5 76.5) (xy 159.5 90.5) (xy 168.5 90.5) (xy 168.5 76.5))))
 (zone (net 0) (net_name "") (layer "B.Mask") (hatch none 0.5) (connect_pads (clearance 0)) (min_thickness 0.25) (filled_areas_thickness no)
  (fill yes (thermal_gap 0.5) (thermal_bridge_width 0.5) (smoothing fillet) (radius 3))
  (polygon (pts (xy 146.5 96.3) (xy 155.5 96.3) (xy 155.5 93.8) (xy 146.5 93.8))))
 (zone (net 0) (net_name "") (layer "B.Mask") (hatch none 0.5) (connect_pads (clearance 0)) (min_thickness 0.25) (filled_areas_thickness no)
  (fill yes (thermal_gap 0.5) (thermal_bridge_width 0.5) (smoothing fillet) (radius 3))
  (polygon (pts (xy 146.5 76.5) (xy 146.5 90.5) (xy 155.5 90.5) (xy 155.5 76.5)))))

